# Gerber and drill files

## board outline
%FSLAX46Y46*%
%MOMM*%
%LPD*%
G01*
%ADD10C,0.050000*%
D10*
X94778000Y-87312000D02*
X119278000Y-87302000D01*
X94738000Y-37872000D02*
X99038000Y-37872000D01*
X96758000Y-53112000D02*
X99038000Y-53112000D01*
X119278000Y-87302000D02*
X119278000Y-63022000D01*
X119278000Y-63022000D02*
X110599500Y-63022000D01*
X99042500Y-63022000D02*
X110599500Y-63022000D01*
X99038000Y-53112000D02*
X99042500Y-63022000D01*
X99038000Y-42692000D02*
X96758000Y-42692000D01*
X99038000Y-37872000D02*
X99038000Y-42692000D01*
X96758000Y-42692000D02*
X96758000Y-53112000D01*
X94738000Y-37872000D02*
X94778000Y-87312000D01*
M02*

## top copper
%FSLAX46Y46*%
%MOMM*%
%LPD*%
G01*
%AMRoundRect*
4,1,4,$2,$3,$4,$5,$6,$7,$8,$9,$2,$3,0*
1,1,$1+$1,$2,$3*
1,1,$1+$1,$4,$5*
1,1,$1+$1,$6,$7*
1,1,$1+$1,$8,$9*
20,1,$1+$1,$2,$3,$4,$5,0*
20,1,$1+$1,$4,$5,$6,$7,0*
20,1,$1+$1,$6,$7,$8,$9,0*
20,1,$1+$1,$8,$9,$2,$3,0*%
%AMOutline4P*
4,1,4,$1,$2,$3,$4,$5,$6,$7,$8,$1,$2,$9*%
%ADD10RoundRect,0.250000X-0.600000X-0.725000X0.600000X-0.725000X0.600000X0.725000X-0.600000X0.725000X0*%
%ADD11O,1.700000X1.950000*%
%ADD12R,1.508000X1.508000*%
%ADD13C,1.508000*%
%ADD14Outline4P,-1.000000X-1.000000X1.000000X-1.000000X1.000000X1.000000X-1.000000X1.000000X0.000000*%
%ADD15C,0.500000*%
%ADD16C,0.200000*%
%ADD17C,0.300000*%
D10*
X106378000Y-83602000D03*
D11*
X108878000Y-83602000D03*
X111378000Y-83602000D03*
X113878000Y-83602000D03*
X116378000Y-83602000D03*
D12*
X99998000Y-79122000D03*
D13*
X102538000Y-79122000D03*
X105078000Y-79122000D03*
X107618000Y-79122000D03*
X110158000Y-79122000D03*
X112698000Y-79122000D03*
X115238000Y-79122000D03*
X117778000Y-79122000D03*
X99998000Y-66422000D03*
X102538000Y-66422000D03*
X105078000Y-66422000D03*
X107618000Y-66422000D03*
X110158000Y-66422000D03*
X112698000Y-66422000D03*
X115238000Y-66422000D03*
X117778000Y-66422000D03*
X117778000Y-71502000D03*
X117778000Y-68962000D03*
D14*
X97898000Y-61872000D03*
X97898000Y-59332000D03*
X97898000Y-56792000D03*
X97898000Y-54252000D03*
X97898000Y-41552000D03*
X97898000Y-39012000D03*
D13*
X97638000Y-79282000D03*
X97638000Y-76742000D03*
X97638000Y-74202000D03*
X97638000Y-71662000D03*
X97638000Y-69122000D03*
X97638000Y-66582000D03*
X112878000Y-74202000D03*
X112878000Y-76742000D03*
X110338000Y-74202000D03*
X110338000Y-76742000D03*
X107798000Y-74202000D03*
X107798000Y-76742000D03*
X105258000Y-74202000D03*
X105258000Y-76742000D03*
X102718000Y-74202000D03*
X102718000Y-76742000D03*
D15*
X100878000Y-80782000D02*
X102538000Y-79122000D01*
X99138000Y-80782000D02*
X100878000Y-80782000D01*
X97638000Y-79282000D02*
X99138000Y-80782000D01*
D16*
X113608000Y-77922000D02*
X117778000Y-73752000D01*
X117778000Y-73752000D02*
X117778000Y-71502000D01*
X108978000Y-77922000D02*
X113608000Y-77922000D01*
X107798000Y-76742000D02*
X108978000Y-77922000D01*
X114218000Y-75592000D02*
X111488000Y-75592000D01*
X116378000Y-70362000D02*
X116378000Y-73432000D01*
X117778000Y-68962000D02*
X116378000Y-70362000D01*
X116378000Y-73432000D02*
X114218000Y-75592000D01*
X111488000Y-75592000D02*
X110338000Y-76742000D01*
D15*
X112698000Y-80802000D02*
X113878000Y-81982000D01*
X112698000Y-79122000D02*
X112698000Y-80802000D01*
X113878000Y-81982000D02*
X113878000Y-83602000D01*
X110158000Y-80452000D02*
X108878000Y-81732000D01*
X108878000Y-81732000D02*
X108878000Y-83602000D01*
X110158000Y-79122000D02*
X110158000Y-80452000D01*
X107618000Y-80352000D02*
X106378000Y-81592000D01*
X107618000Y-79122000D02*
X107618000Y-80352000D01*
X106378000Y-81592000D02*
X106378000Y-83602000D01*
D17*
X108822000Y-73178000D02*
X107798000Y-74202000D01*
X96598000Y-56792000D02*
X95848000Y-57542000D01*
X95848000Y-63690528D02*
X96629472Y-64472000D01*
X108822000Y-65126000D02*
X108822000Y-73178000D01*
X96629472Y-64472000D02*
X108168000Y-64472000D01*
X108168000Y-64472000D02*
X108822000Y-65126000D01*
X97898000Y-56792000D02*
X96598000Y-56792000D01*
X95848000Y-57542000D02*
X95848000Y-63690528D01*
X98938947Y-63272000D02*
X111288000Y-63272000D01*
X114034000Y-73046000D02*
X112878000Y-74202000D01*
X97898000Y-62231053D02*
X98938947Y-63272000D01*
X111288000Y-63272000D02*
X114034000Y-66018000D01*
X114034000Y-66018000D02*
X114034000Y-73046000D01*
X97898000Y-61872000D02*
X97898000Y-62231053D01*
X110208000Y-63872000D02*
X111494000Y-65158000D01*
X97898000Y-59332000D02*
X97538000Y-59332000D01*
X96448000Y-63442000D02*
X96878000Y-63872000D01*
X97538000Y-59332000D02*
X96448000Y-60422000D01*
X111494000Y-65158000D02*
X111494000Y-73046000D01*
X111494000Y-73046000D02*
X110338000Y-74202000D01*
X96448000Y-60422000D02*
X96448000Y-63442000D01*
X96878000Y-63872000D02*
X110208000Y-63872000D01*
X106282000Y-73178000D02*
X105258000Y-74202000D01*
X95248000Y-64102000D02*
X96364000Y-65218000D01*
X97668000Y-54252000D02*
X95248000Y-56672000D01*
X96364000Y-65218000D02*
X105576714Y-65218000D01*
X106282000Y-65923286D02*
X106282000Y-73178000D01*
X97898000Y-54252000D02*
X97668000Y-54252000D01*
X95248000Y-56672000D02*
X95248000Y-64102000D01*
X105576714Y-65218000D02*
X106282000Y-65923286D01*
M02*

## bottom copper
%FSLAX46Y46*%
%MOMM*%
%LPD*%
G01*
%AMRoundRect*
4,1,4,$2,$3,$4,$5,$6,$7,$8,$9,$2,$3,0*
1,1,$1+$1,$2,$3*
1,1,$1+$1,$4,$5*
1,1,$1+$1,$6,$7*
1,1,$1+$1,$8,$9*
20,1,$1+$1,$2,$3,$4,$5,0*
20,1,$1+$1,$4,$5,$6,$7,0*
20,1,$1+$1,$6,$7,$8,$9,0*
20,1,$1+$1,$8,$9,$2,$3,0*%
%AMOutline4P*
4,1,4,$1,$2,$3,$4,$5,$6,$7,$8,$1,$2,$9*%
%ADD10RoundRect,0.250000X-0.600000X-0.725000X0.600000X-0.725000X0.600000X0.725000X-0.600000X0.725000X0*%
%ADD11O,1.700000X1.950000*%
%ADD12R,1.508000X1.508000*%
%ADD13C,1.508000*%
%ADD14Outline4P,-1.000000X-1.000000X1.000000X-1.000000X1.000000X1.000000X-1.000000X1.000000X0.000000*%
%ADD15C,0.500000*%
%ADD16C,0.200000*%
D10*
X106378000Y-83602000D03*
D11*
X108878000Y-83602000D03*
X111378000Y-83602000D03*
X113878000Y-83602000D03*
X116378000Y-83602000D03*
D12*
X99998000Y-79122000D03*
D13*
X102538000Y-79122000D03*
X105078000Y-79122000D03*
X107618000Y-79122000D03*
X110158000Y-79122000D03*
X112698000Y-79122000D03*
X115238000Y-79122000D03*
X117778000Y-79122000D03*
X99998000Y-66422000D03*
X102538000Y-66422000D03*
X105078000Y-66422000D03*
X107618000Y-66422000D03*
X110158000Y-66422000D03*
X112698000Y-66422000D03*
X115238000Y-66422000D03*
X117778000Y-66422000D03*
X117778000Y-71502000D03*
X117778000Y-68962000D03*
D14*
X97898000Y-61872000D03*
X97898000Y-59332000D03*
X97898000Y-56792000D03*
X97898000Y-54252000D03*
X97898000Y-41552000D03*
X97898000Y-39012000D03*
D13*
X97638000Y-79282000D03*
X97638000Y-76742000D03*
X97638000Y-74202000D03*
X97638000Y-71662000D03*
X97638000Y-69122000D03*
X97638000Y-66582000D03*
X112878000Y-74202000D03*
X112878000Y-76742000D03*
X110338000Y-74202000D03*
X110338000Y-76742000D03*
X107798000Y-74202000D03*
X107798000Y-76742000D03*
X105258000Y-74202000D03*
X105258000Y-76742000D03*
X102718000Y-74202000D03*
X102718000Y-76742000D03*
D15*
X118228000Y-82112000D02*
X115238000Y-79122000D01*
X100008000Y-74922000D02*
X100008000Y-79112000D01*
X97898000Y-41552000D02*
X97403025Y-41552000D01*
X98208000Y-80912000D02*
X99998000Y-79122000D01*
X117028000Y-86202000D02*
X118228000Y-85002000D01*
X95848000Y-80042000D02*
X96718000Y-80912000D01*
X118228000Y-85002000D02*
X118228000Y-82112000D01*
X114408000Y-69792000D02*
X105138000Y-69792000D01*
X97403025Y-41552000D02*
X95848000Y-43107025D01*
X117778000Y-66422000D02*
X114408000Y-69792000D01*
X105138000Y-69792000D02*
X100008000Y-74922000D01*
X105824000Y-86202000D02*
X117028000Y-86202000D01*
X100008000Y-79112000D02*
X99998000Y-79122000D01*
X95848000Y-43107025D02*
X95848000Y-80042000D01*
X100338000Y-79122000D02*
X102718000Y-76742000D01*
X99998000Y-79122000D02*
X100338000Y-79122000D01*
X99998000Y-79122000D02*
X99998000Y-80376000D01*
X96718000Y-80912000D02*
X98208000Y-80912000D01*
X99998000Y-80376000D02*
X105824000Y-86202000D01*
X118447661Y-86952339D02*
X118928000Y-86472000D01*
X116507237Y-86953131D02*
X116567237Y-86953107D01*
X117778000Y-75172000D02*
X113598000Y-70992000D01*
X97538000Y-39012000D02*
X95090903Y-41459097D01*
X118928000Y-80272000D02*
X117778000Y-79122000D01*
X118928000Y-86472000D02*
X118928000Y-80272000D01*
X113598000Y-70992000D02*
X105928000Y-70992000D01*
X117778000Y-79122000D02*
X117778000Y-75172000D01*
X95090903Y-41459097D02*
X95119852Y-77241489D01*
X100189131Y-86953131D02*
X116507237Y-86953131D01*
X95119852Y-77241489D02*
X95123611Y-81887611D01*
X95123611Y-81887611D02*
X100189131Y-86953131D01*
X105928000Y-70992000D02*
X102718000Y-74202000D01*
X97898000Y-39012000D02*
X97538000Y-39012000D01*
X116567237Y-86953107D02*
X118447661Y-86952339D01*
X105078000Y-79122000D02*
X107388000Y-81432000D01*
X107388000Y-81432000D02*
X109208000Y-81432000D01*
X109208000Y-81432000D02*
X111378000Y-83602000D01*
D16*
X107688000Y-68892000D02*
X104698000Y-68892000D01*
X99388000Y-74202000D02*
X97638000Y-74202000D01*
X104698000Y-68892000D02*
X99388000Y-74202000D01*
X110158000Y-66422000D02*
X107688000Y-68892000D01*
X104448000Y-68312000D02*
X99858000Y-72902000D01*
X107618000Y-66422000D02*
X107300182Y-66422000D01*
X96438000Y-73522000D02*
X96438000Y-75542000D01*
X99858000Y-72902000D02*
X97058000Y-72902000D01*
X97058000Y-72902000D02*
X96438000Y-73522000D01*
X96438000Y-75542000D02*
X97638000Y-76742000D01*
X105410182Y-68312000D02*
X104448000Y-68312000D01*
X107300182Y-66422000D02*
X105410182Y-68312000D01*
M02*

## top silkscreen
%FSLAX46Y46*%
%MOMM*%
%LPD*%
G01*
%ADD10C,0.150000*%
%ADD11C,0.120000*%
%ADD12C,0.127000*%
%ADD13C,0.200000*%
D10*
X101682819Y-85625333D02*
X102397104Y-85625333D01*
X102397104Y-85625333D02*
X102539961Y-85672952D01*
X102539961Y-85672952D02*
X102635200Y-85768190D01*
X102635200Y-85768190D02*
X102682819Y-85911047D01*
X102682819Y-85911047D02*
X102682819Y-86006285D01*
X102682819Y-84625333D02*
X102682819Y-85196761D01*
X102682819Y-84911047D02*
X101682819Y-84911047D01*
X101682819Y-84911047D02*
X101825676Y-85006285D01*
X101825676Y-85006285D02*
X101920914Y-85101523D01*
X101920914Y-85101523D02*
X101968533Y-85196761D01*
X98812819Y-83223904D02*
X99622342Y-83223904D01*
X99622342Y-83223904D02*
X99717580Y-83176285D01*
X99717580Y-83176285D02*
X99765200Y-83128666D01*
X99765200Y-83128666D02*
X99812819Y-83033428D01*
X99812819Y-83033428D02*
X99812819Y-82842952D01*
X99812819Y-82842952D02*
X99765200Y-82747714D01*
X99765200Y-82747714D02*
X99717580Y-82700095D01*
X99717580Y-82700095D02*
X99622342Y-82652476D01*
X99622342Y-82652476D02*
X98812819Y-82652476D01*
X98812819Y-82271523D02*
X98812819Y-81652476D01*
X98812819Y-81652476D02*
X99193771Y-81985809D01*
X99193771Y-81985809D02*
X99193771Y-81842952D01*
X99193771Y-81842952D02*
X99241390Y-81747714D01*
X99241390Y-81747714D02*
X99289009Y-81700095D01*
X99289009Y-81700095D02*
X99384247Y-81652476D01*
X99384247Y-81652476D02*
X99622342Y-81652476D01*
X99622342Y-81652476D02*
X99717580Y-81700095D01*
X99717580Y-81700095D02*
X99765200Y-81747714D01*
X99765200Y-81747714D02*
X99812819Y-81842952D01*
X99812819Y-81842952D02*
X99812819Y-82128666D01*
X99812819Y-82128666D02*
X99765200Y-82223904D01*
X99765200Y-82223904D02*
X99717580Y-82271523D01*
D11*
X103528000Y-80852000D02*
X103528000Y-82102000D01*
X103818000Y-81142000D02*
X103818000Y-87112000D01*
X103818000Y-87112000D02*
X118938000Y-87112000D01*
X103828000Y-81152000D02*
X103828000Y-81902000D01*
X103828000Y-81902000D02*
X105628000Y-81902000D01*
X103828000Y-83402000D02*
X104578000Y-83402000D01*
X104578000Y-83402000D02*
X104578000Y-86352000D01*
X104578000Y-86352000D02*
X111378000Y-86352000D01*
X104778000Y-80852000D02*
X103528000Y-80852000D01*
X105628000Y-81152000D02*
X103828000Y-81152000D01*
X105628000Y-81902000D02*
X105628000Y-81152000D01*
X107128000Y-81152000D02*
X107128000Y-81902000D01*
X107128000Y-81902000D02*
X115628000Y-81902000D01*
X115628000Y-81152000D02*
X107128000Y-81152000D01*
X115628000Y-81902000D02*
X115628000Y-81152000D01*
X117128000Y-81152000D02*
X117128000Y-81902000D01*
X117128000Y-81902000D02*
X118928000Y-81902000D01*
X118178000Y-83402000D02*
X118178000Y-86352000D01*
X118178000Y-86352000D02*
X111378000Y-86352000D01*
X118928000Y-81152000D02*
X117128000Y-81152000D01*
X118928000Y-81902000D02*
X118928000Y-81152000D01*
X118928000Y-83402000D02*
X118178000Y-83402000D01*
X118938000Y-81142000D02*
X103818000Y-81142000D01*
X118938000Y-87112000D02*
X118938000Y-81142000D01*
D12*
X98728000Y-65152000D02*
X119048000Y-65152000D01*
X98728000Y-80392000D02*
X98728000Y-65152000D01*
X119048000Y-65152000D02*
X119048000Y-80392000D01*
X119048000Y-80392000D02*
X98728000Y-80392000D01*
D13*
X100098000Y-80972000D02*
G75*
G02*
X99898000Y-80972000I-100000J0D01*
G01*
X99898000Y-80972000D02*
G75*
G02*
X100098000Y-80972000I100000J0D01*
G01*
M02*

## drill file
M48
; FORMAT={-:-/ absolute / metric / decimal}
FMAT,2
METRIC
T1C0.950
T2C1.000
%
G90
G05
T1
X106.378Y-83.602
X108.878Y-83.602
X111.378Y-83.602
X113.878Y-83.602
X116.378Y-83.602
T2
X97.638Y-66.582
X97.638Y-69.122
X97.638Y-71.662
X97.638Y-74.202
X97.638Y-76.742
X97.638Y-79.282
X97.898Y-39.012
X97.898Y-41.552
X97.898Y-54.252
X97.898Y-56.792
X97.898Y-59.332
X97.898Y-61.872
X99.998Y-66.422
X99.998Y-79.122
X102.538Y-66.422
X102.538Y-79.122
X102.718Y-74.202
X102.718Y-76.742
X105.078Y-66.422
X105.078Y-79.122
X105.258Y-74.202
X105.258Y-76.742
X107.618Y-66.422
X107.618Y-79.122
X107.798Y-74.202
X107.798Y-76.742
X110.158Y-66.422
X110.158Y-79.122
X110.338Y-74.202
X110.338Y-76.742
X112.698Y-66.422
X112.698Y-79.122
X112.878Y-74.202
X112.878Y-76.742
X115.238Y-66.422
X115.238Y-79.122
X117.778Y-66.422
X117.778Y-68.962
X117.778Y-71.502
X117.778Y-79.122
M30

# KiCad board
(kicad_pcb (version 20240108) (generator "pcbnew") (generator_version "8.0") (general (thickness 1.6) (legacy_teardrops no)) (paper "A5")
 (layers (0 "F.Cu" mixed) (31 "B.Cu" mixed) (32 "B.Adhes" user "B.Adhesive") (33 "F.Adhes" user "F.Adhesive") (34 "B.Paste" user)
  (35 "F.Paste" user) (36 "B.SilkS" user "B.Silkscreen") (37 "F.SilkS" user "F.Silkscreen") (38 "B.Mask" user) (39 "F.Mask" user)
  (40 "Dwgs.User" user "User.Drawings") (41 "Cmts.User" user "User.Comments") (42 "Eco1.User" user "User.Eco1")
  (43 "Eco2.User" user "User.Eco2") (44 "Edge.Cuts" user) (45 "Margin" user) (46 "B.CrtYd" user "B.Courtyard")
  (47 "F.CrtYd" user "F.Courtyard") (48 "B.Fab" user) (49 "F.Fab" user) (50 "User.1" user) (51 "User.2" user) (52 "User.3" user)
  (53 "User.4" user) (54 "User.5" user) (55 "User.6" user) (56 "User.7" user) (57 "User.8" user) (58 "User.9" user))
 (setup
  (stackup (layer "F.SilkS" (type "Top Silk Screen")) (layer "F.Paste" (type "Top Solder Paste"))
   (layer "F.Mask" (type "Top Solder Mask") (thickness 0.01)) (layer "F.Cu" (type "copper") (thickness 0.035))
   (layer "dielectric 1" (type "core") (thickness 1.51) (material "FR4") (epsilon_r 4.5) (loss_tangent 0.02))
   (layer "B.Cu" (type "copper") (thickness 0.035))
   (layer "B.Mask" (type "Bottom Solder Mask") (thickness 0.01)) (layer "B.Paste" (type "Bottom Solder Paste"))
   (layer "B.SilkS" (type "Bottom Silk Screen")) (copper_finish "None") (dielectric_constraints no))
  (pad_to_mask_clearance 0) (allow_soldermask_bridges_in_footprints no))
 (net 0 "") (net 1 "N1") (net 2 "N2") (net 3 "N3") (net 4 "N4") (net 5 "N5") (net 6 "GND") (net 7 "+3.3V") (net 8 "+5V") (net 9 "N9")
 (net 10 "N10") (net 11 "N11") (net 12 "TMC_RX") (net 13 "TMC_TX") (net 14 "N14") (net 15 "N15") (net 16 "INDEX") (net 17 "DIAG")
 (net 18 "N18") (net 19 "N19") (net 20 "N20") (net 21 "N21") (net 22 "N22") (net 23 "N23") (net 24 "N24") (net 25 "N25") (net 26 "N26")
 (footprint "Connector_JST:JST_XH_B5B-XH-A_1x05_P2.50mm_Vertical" (layer "F.Cu") (at 106.378 83.602)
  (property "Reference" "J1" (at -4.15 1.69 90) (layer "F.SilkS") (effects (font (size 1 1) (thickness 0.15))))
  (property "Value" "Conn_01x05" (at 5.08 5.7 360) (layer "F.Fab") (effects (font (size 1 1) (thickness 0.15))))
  (fp_line (start -2.85 -2.75) (end -2.85 -1.5) (stroke (width 0.12) (type solid)) (layer "F.SilkS"))
  (fp_line (start -2.56 -2.46) (end -2.56 3.51) (stroke (width 0.12) (type solid)) (layer "F.SilkS"))
  (fp_line (start -2.56 3.51) (end 12.56 3.51) (stroke (width 0.12) (type solid)) (layer "F.SilkS"))
  (fp_line (start -2.55 -2.45) (end -2.55 -1.7) (stroke (width 0.12) (type solid)) (layer "F.SilkS"))
  (fp_line (start -2.55 -1.7) (end -0.75 -1.7) (stroke (width 0.12) (type solid)) (layer "F.SilkS"))
  (fp_line (start -2.55 -0.2) (end -1.8 -0.2) (stroke (width 0.12) (type solid)) (layer "F.SilkS"))
  (fp_line (start -1.8 -0.2) (end -1.8 2.75) (stroke (width 0.12) (type solid)) (layer "F.SilkS"))
  (fp_line (start -1.8 2.75) (end 5 2.75) (stroke (width 0.12) (type solid)) (layer "F.SilkS"))
  (fp_line (start -1.6 -2.75) (end -2.85 -2.75) (stroke (width 0.12) (type solid)) (layer "F.SilkS"))
  (fp_line (start -0.75 -2.45) (end -2.55 -2.45) (stroke (width 0.12) (type solid)) (layer "F.SilkS"))
  (fp_line (start -0.75 -1.7) (end -0.75 -2.45) (stroke (width 0.12) (type solid)) (layer "F.SilkS"))
  (fp_line (start 0.75 -2.45) (end 0.75 -1.7) (stroke (width 0.12) (type solid)) (layer "F.SilkS"))
  (fp_line (start 0.75 -1.7) (end 9.25 -1.7) (stroke (width 0.12) (type solid)) (layer "F.SilkS"))
  (fp_line (start 9.25 -2.45) (end 0.75 -2.45) (stroke (width 0.12) (type solid)) (layer "F.SilkS"))
  (fp_line (start 9.25 -1.7) (end 9.25 -2.45) (stroke (width 0.12) (type solid)) (layer "F.SilkS"))
  (fp_line (start 10.75 -2.45) (end 10.75 -1.7) (stroke (width 0.12) (type solid)) (layer "F.SilkS"))
  (fp_line (start 10.75 -1.7) (end 12.55 -1.7) (stroke (width 0.12) (type solid)) (layer "F.SilkS"))
  (fp_line (start 11.8 -0.2) (end 11.8 2.75) (stroke (width 0.12) (type solid)) (layer "F.SilkS"))
  (fp_line (start 11.8 2.75) (end 5 2.75) (stroke (width 0.12) (type solid)) (layer "F.SilkS"))
  (fp_line (start 12.55 -2.45) (end 10.75 -2.45) (stroke (width 0.12) (type solid)) (layer "F.SilkS"))
  (fp_line (start 12.55 -1.7) (end 12.55 -2.45) (stroke (width 0.12) (type solid)) (layer "F.SilkS"))
  (fp_line (start 12.55 -0.2) (end 11.8 -0.2) (stroke (width 0.12) (type solid)) (layer "F.SilkS"))
  (fp_line (start 12.56 -2.46) (end -2.56 -2.46) (stroke (width 0.12) (type solid)) (layer "F.SilkS"))
  (fp_line (start 12.56 3.51) (end 12.56 -2.46) (stroke (width 0.12) (type solid)) (layer "F.SilkS"))
  (pad "1" thru_hole roundrect (at 0 0) (size 1.7 1.95) (drill 0.95) (layers "*.Cu" "*.Mask") (remove_unused_layers no)
   (roundrect_rratio 0.147059) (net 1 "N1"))
  (pad "2" thru_hole oval (at 2.5 0) (size 1.7 1.95) (drill 0.95) (layers "*.Cu" "*.Mask") (remove_unused_layers no) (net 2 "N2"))
  (pad "3" thru_hole oval (at 5 0) (size 1.7 1.95) (drill 0.95) (layers "*.Cu" "*.Mask") (remove_unused_layers no) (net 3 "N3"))
  (pad "4" thru_hole oval (at 7.5 0) (size 1.7 1.95) (drill 0.95) (layers "*.Cu" "*.Mask") (remove_unused_layers no) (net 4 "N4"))
  (pad "5" thru_hole oval (at 10 0) (size 1.7 1.95) (drill 0.95) (layers "*.Cu" "*.Mask") (remove_unused_layers no) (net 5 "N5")))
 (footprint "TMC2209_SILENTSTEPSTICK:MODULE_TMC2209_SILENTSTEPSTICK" (layer "F.Cu") (at 108.888 72.772 90)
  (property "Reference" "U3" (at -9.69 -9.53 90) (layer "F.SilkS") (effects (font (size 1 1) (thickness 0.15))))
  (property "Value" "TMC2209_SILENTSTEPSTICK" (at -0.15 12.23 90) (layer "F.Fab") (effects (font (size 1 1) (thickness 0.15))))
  (fp_line (start 7.62 -10.16) (end 7.62 10.16) (stroke (width 0.127) (type solid)) (layer "F.SilkS"))
  (fp_line (start -7.62 -10.16) (end 7.62 -10.16) (stroke (width 0.127) (type solid)) (layer "F.SilkS"))
  (fp_line (start 7.62 10.16) (end -7.62 10.16) (stroke (width 0.127) (type solid)) (layer "F.SilkS"))
  (fp_line (start -7.62 10.16) (end -7.62 -10.16) (stroke (width 0.127) (type solid)) (layer "F.SilkS"))
  (fp_circle (center -8.2 -8.89) (end -8.1 -8.89) (stroke (width 0.2) (type solid)) (fill none) (layer "F.SilkS"))
  (pad "1" thru_hole rect (at -6.35 -8.89 90) (size 1.508 1.508) (drill 1) (layers "*.Cu" "*.Mask") (remove_unused_layers no) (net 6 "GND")
   (solder_mask_margin 0.102))
  (pad "2" thru_hole circle (at -6.35 -6.35 90) (size 1.508 1.508) (drill 1) (layers "*.Cu" "*.Mask") (remove_unused_layers no)
   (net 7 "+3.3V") (solder_mask_margin 0.102))
  (pad "3" thru_hole circle (at -6.35 -3.81 90) (size 1.508 1.508) (drill 1) (layers "*.Cu" "*.Mask") (remove_unused_layers no) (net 3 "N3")
   (solder_mask_margin 0.102))
  (pad "4" thru_hole circle (at -6.35 -1.27 90) (size 1.508 1.508) (drill 1) (layers "*.Cu" "*.Mask") (remove_unused_layers no) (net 1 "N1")
   (solder_mask_margin 0.102))
  (pad "5" thru_hole circle (at -6.35 1.27 90) (size 1.508 1.508) (drill 1) (layers "*.Cu" "*.Mask") (remove_unused_layers no) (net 2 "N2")
   (solder_mask_margin 0.102))
  (pad "6" thru_hole circle (at -6.35 3.81 90) (size 1.508 1.508) (drill 1) (layers "*.Cu" "*.Mask") (remove_unused_layers no) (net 4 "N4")
   (solder_mask_margin 0.102))
  (pad "7" thru_hole circle (at -6.35 6.35 90) (size 1.508 1.508) (drill 1) (layers "*.Cu" "*.Mask") (remove_unused_layers no) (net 6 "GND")
   (solder_mask_margin 0.102))
  (pad "8" thru_hole circle (at -6.35 8.89 90) (size 1.508 1.508) (drill 1) (layers "*.Cu" "*.Mask") (remove_unused_layers no) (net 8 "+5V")
   (solder_mask_margin 0.102))
  (pad "9" thru_hole circle (at 6.35 -8.89 90) (size 1.508 1.508) (drill 1) (layers "*.Cu" "*.Mask") (remove_unused_layers no) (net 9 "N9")
   (solder_mask_margin 0.102))
  (pad "10" thru_hole circle (at 6.35 -6.35 90) (size 1.508 1.508) (drill 1) (layers "*.Cu" "*.Mask") (remove_unused_layers no)
   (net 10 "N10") (solder_mask_margin 0.102))
  (pad "11" thru_hole circle (at 6.35 -3.81 90) (size 1.508 1.508) (drill 1) (layers "*.Cu" "*.Mask") (remove_unused_layers no)
   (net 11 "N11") (solder_mask_margin 0.102))
  (pad "12" thru_hole circle (at 6.35 -1.27 90) (size 1.508 1.508) (drill 1) (layers "*.Cu" "*.Mask") (remove_unused_layers no)
   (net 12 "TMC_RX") (solder_mask_margin 0.102))
  (pad "13" thru_hole circle (at 6.35 1.27 90) (size 1.508 1.508) (drill 1) (layers "*.Cu" "*.Mask") (remove_unused_layers no)
   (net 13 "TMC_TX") (solder_mask_margin 0.102))
  (pad "14" thru_hole circle (at 6.35 3.81 90) (size 1.508 1.508) (drill 1) (layers "*.Cu" "*.Mask") (remove_unused_layers no)
   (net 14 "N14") (solder_mask_margin 0.102))
  (pad "15" thru_hole circle (at 6.35 6.35 90) (size 1.508 1.508) (drill 1) (layers "*.Cu" "*.Mask") (remove_unused_layers no)
   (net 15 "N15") (solder_mask_margin 0.102))
  (pad "16" thru_hole circle (at 6.35 8.89 90) (size 1.508 1.508) (drill 1) (layers "*.Cu" "*.Mask") (remove_unused_layers no) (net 6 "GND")
   (solder_mask_margin 0.102))
  (pad "17" thru_hole circle (at 1.27 8.89 90) (size 1.508 1.508) (drill 1) (layers "*.Cu" "*.Mask") (remove_unused_layers no)
   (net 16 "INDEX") (solder_mask_margin 0.102))
  (pad "18" thru_hole circle (at 3.81 8.89 90) (size 1.508 1.508) (drill 1) (layers "*.Cu" "*.Mask") (remove_unused_layers no)
   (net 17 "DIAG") (solder_mask_margin 0.102)))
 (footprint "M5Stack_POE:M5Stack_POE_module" (layer "B.Cu") (at 97.898 61.872)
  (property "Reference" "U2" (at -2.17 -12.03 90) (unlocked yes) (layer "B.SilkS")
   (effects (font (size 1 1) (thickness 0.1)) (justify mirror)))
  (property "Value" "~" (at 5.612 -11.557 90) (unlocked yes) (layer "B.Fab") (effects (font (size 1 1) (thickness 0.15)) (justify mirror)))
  (pad "1" thru_hole trapezoid (at 0 0) (size 2 2) (drill 1) (layers "*.Cu" "*.Mask") (remove_unused_layers no) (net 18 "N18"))
  (pad "2" thru_hole trapezoid (at 0 -2.54) (size 2 2) (drill 1) (layers "*.Cu" "*.Mask") (remove_unused_layers no) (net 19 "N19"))
  (pad "3" thru_hole trapezoid (at 0 -5.08) (size 2 2) (drill 1) (layers "*.Cu" "*.Mask") (remove_unused_layers no) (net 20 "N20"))
  (pad "4" thru_hole trapezoid (at 0 -7.62) (size 2 2) (drill 1) (layers "*.Cu" "*.Mask") (remove_unused_layers no) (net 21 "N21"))
  (pad "5" thru_hole trapezoid (at 0 -20.32) (size 2 2) (drill 1) (layers "*.Cu" "*.Mask") (remove_unused_layers no) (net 6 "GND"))
  (pad "6" thru_hole trapezoid (at 0 -22.86) (size 2 2) (drill 1) (layers "*.Cu" "*.Mask") (remove_unused_layers no) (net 8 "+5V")))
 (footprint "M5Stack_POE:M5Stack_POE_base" (layer "B.Cu") (at 107.798 74.202 180)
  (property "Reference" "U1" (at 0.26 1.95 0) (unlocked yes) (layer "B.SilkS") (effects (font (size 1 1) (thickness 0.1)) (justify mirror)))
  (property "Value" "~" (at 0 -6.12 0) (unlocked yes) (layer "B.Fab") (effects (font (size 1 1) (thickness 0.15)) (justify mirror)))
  (pad "a1" thru_hole circle (at 10.16 -5.08 180) (size 1.508 1.508) (drill 1) (layers "*.Cu" "*.Mask") (remove_unused_layers no)
   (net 7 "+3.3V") (solder_mask_margin 0.102))
  (pad "a2" thru_hole circle (at 10.16 -2.54 180) (size 1.508 1.508) (drill 1) (layers "*.Cu" "*.Mask") (remove_unused_layers no)
   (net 12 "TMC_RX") (solder_mask_margin 0.102))
  (pad "a3" thru_hole circle (at 10.16 0 180) (size 1.508 1.508) (drill 1) (layers "*.Cu" "*.Mask") (remove_unused_layers no)
   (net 13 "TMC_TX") (solder_mask_margin 0.102))
  (pad "a4" thru_hole circle (at 10.16 2.54 180) (size 1.508 1.508) (drill 1) (layers "*.Cu" "*.Mask") (remove_unused_layers no)
   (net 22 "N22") (solder_mask_margin 0.102))
  (pad "a5" thru_hole circle (at 10.16 5.08 180) (size 1.508 1.508) (drill 1) (layers "*.Cu" "*.Mask") (remove_unused_layers no)
   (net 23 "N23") (solder_mask_margin 0.102))
  (pad "a6" thru_hole circle (at 10.16 7.62 180) (size 1.508 1.508) (drill 1) (layers "*.Cu" "*.Mask") (remove_unused_layers no)
   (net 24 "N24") (solder_mask_margin 0.102))
  (pad "b1" thru_hole circle (at -5.08 0 180) (size 1.508 1.508) (drill 1) (layers "*.Cu" "*.Mask") (remove_unused_layers no) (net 18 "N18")
   (solder_mask_margin 0.102))
  (pad "b2" thru_hole circle (at -5.08 -2.54 180) (size 1.508 1.508) (drill 1) (layers "*.Cu" "*.Mask") (remove_unused_layers no)
   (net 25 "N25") (solder_mask_margin 0.102))
  (pad "b3" thru_hole circle (at -2.54 0 180) (size 1.508 1.508) (drill 1) (layers "*.Cu" "*.Mask") (remove_unused_layers no) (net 19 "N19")
   (solder_mask_margin 0.102))
  (pad "b4" thru_hole circle (at -2.54 -2.54 180) (size 1.508 1.508) (drill 1) (layers "*.Cu" "*.Mask") (remove_unused_layers no)
   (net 17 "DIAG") (solder_mask_margin 0.102))
  (pad "b5" thru_hole circle (at 0 0 180) (size 1.508 1.508) (drill 1) (layers "*.Cu" "*.Mask") (remove_unused_layers no) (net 20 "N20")
   (solder_mask_margin 0.102))
  (pad "b6" thru_hole circle (at 0 -2.54 180) (size 1.508 1.508) (drill 1) (layers "*.Cu" "*.Mask") (remove_unused_layers no)
   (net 16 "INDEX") (solder_mask_margin 0.102))
  (pad "b7" thru_hole circle (at 2.54 0 180) (size 1.508 1.508) (drill 1) (layers "*.Cu" "*.Mask") (remove_unused_layers no) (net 21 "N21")
   (solder_mask_margin 0.102))
  (pad "b8" thru_hole circle (at 2.54 -2.54 180) (size 1.508 1.508) (drill 1) (layers "*.Cu" "*.Mask") (remove_unused_layers no)
   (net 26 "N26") (solder_mask_margin 0.102))
  (pad "b9" thru_hole circle (at 5.08 0 180) (size 1.508 1.508) (drill 1) (layers "*.Cu" "*.Mask") (remove_unused_layers no) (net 8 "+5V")
   (solder_mask_margin 0.102))
  (pad "b10" thru_hole circle (at 5.08 -2.54 180) (size 1.508 1.508) (drill 1) (layers "*.Cu" "*.Mask") (remove_unused_layers no)
   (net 6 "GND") (solder_mask_margin 0.102)))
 (gr_line (start 94.778 87.312) (end 119.278 87.302) (stroke (width 0.05) (type default)) (layer "Edge.Cuts"))
 (gr_line (start 94.738 37.872) (end 99.038 37.872) (stroke (width 0.05) (type default)) (layer "Edge.Cuts"))
 (gr_line (start 96.758 53.112) (end 99.038 53.112) (stroke (width 0.05) (type default)) (layer "Edge.Cuts"))
 (gr_line (start 119.278 87.302) (end 119.278 63.022) (stroke (width 0.05) (type default)) (layer "Edge.Cuts"))
 (gr_line (start 119.278 63.022) (end 110.5995 63.022) (stroke (width 0.05) (type default)) (layer "Edge.Cuts"))
 (gr_line (start 99.0425 63.022) (end 110.5995 63.022) (stroke (width 0.05) (type default)) (layer "Edge.Cuts"))
 (gr_line (start 99.038 53.112) (end 99.0425 63.022) (stroke (width 0.05) (type default)) (layer "Edge.Cuts"))
 (gr_line (start 99.038 42.692) (end 96.758 42.692) (stroke (width 0.05) (type default)) (layer "Edge.Cuts"))
 (gr_line (start 99.038 37.872) (end 99.038 42.692) (stroke (width 0.05) (type default)) (layer "Edge.Cuts"))
 (gr_line (start 96.758 42.692) (end 96.758 53.112) (stroke (width 0.05) (type default)) (layer "Edge.Cuts"))
 (gr_line (start 94.738 37.872) (end 94.778 87.312) (stroke (width 0.05) (type default)) (layer "Edge.Cuts"))
 (segment (start 100.878 80.782) (end 102.538 79.122) (width 0.5) (layer "F.Cu") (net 7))
 (segment (start 99.138 80.782) (end 100.878 80.782) (width 0.5) (layer "F.Cu") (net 7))
 (segment (start 97.638 79.282) (end 99.138 80.782) (width 0.5) (layer "F.Cu") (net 7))
 (segment (start 118.228 82.112) (end 115.238 79.122) (width 0.5) (layer "B.Cu") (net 6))
 (segment (start 100.008 74.922) (end 100.008 79.112) (width 0.5) (layer "B.Cu") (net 6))
 (segment (start 97.898 41.552) (end 97.403025 41.552) (width 0.5) (layer "B.Cu") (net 6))
 (segment (start 98.208 80.912) (end 99.998 79.122) (width 0.5) (layer "B.Cu") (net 6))
 (segment (start 117.028 86.202) (end 118.228 85.002) (width 0.5) (layer "B.Cu") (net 6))
 (segment (start 95.848 80.042) (end 96.718 80.912) (width 0.5) (layer "B.Cu") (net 6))
 (segment (start 118.228 85.002) (end 118.228 82.112) (width 0.5) (layer "B.Cu") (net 6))
 (segment (start 114.408 69.792) (end 105.138 69.792) (width 0.5) (layer "B.Cu") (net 6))
 (segment (start 97.403025 41.552) (end 95.848 43.107025) (width 0.5) (layer "B.Cu") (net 6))
 (segment (start 117.778 66.422) (end 114.408 69.792) (width 0.5) (layer "B.Cu") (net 6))
 (segment (start 105.138 69.792) (end 100.008 74.922) (width 0.5) (layer "B.Cu") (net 6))
 (segment (start 105.824 86.202) (end 117.028 86.202) (width 0.5) (layer "B.Cu") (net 6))
 (segment (start 100.008 79.112) (end 99.998 79.122) (width 0.5) (layer "B.Cu") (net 6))
 (segment (start 95.848 43.107025) (end 95.848 80.042) (width 0.5) (layer "B.Cu") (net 6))
 (segment (start 100.338 79.122) (end 102.718 76.742) (width 0.5) (layer "B.Cu") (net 6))
 (segment (start 99.998 79.122) (end 100.338 79.122) (width 0.5) (layer "B.Cu") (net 6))
 (segment (start 99.998 79.122) (end 99.998 80.376) (width 0.5) (layer "B.Cu") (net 6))
 (segment (start 96.718 80.912) (end 98.208 80.912) (width 0.5) (layer "B.Cu") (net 6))
 (segment (start 99.998 80.376) (end 105.824 86.202) (width 0.5) (layer "B.Cu") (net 6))
 (segment (start 118.447661 86.952339) (end 118.928 86.472) (width 0.5) (layer "B.Cu") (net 8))
 (segment (start 116.507237 86.953131) (end 116.567237 86.953107) (width 0.5) (layer "B.Cu") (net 8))
 (segment (start 117.778 75.172) (end 113.598 70.992) (width 0.5) (layer "B.Cu") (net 8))
 (segment (start 97.538 39.012) (end 95.090903 41.459097) (width 0.5) (layer "B.Cu") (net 8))
 (segment (start 118.928 80.272) (end 117.778 79.122) (width 0.5) (layer "B.Cu") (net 8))
 (segment (start 118.928 86.472) (end 118.928 80.272) (width 0.5) (layer "B.Cu") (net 8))
 (segment (start 113.598 70.992) (end 105.928 70.992) (width 0.5) (layer "B.Cu") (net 8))
 (segment (start 117.778 79.122) (end 117.778 75.172) (width 0.5) (layer "B.Cu") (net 8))
 (segment (start 95.090903 41.459097) (end 95.119852 77.241489) (width 0.5) (layer "B.Cu") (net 8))
 (segment (start 100.189131 86.953131) (end 116.507237 86.953131) (width 0.5) (layer "B.Cu") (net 8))
 (segment (start 95.119852 77.241489) (end 95.123611 81.887611) (width 0.5) (layer "B.Cu") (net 8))
 (segment (start 95.123611 81.887611) (end 100.189131 86.953131) (width 0.5) (layer "B.Cu") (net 8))
 (segment (start 105.928 70.992) (end 102.718 74.202) (width 0.5) (layer "B.Cu") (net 8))
 (segment (start 97.898 39.012) (end 97.538 39.012) (width 0.5) (layer "B.Cu") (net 8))
 (segment (start 116.567237 86.953107) (end 118.447661 86.952339) (width 0.5) (layer "B.Cu") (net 8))
 (segment (start 113.608 77.922) (end 117.778 73.752) (width 0.2) (layer "F.Cu") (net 16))
 (segment (start 117.778 73.752) (end 117.778 71.502) (width 0.2) (layer "F.Cu") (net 16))
 (segment (start 108.978 77.922) (end 113.608 77.922) (width 0.2) (layer "F.Cu") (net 16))
 (segment (start 107.798 76.742) (end 108.978 77.922) (width 0.2) (layer "F.Cu") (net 16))
 (segment (start 114.218 75.592) (end 111.488 75.592) (width 0.2) (layer "F.Cu") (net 17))
 (segment (start 116.378 70.362) (end 116.378 73.432) (width 0.2) (layer "F.Cu") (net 17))
 (segment (start 117.778 68.962) (end 116.378 70.362) (width 0.2) (layer "F.Cu") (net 17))
 (segment (start 116.378 73.432) (end 114.218 75.592) (width 0.2) (layer "F.Cu") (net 17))
 (segment (start 111.488 75.592) (end 110.338 76.742) (width 0.2) (layer "F.Cu") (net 17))
 (segment (start 112.698 80.802) (end 113.878 81.982) (width 0.5) (layer "F.Cu") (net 4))
 (segment (start 112.698 79.122) (end 112.698 80.802) (width 0.5) (layer "F.Cu") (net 4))
 (segment (start 113.878 81.982) (end 113.878 83.602) (width 0.5) (layer "F.Cu") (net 4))
 (segment (start 110.158 80.452) (end 108.878 81.732) (width 0.5) (layer "F.Cu") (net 2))
 (segment (start 108.878 81.732) (end 108.878 83.602) (width 0.5) (layer "F.Cu") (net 2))
 (segment (start 110.158 79.122) (end 110.158 80.452) (width 0.5) (layer "F.Cu") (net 2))
 (segment (start 107.618 80.352) (end 106.378 81.592) (width 0.5) (layer "F.Cu") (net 1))
 (segment (start 107.618 79.122) (end 107.618 80.352) (width 0.5) (layer "F.Cu") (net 1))
 (segment (start 106.378 81.592) (end 106.378 83.602) (width 0.5) (layer "F.Cu") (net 1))
 (segment (start 105.078 79.122) (end 107.388 81.432) (width 0.5) (layer "B.Cu") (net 3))
 (segment (start 107.388 81.432) (end 109.208 81.432) (width 0.5) (layer "B.Cu") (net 3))
 (segment (start 109.208 81.432) (end 111.378 83.602) (width 0.5) (layer "B.Cu") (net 3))
 (segment (start 107.688 68.892) (end 104.698 68.892) (width 0.2) (layer "B.Cu") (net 13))
 (segment (start 99.388 74.202) (end 97.638 74.202) (width 0.2) (layer "B.Cu") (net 13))
 (segment (start 104.698 68.892) (end 99.388 74.202) (width 0.2) (layer "B.Cu") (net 13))
 (segment (start 110.158 66.422) (end 107.688 68.892) (width 0.2) (layer "B.Cu") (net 13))
 (segment (start 104.448 68.312) (end 99.858 72.902) (width 0.2) (layer "B.Cu") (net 12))
 (segment (start 107.618 66.422) (end 107.300182 66.422) (width 0.2) (layer "B.Cu") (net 12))
 (segment (start 96.438 73.522) (end 96.438 75.542) (width 0.2) (layer "B.Cu") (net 12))
 (segment (start 99.858 72.902) (end 97.058 72.902) (width 0.2) (layer "B.Cu") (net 12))
 (segment (start 97.058 72.902) (end 96.438 73.522) (width 0.2) (layer "B.Cu") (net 12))
 (segment (start 96.438 75.542) (end 97.638 76.742) (width 0.2) (layer "B.Cu") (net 12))
 (segment (start 105.410182 68.312) (end 104.448 68.312) (width 0.2) (layer "B.Cu") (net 12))
 (segment (start 107.300182 66.422) (end 105.410182 68.312) (width 0.2) (layer "B.Cu") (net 12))
 (segment (start 108.822 73.178) (end 107.798 74.202) (width 0.3) (layer "F.Cu") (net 20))
 (segment (start 96.598 56.792) (end 95.848 57.542) (width 0.3) (layer "F.Cu") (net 20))
 (segment (start 95.848 63.690528) (end 96.629472 64.472) (width 0.3) (layer "F.Cu") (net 20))
 (segment (start 108.822 65.126) (end 108.822 73.178) (width 0.3) (layer "F.Cu") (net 20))
 (segment (start 96.629472 64.472) (end 108.168 64.472) (width 0.3) (layer "F.Cu") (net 20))
 (segment (start 108.168 64.472) (end 108.822 65.126) (width 0.3) (layer "F.Cu") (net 20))
 (segment (start 97.898 56.792) (end 96.598 56.792) (width 0.3) (layer "F.Cu") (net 20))
 (segment (start 95.848 57.542) (end 95.848 63.690528) (width 0.3) (layer "F.Cu") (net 20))
 (segment (start 98.938947 63.272) (end 111.288 63.272) (width 0.3) (layer "F.Cu") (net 18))
 (segment (start 114.034 73.046) (end 112.878 74.202) (width 0.3) (layer "F.Cu") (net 18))
 (segment (start 97.898 62.231053) (end 98.938947 63.272) (width 0.3) (layer "F.Cu") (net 18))
 (segment (start 111.288 63.272) (end 114.034 66.018) (width 0.3) (layer "F.Cu") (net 18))
 (segment (start 114.034 66.018) (end 114.034 73.046) (width 0.3) (layer "F.Cu") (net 18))
 (segment (start 97.898 61.872) (end 97.898 62.231053) (width 0.3) (layer "F.Cu") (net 18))
 (segment (start 110.208 63.872) (end 111.494 65.158) (width 0.3) (layer "F.Cu") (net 19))
 (segment (start 97.898 59.332) (end 97.538 59.332) (width 0.3) (layer "F.Cu") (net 19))
 (segment (start 96.448 63.442) (end 96.878 63.872) (width 0.3) (layer "F.Cu") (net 19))
 (segment (start 97.538 59.332) (end 96.448 60.422) (width 0.3) (layer "F.Cu") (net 19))
 (segment (start 111.494 65.158) (end 111.494 73.046) (width 0.3) (layer "F.Cu") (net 19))
 (segment (start 111.494 73.046) (end 110.338 74.202) (width 0.3) (layer "F.Cu") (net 19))
 (segment (start 96.448 60.422) (end 96.448 63.442) (width 0.3) (layer "F.Cu") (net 19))
 (segment (start 96.878 63.872) (end 110.208 63.872) (width 0.3) (layer "F.Cu") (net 19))
 (segment (start 106.282 73.178) (end 105.258 74.202) (width 0.3) (layer "F.Cu") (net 21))
 (segment (start 95.248 64.102) (end 96.364 65.218) (width 0.3) (layer "F.Cu") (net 21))
 (segment (start 97.668 54.252) (end 95.248 56.672) (width 0.3) (layer "F.Cu") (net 21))
 (segment (start 96.364 65.218) (end 105.576714 65.218) (width 0.3) (layer "F.Cu") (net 21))
 (segment (start 106.282 65.923286) (end 106.282 73.178) (width 0.3) (layer "F.Cu") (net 21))
 (segment (start 97.898 54.252) (end 97.668 54.252) (width 0.3) (layer "F.Cu") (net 21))
 (segment (start 95.248 56.672) (end 95.248 64.102) (width 0.3) (layer "F.Cu") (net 21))
 (segment (start 105.576714 65.218) (end 106.282 65.923286) (width 0.3) (layer "F.Cu") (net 21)))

